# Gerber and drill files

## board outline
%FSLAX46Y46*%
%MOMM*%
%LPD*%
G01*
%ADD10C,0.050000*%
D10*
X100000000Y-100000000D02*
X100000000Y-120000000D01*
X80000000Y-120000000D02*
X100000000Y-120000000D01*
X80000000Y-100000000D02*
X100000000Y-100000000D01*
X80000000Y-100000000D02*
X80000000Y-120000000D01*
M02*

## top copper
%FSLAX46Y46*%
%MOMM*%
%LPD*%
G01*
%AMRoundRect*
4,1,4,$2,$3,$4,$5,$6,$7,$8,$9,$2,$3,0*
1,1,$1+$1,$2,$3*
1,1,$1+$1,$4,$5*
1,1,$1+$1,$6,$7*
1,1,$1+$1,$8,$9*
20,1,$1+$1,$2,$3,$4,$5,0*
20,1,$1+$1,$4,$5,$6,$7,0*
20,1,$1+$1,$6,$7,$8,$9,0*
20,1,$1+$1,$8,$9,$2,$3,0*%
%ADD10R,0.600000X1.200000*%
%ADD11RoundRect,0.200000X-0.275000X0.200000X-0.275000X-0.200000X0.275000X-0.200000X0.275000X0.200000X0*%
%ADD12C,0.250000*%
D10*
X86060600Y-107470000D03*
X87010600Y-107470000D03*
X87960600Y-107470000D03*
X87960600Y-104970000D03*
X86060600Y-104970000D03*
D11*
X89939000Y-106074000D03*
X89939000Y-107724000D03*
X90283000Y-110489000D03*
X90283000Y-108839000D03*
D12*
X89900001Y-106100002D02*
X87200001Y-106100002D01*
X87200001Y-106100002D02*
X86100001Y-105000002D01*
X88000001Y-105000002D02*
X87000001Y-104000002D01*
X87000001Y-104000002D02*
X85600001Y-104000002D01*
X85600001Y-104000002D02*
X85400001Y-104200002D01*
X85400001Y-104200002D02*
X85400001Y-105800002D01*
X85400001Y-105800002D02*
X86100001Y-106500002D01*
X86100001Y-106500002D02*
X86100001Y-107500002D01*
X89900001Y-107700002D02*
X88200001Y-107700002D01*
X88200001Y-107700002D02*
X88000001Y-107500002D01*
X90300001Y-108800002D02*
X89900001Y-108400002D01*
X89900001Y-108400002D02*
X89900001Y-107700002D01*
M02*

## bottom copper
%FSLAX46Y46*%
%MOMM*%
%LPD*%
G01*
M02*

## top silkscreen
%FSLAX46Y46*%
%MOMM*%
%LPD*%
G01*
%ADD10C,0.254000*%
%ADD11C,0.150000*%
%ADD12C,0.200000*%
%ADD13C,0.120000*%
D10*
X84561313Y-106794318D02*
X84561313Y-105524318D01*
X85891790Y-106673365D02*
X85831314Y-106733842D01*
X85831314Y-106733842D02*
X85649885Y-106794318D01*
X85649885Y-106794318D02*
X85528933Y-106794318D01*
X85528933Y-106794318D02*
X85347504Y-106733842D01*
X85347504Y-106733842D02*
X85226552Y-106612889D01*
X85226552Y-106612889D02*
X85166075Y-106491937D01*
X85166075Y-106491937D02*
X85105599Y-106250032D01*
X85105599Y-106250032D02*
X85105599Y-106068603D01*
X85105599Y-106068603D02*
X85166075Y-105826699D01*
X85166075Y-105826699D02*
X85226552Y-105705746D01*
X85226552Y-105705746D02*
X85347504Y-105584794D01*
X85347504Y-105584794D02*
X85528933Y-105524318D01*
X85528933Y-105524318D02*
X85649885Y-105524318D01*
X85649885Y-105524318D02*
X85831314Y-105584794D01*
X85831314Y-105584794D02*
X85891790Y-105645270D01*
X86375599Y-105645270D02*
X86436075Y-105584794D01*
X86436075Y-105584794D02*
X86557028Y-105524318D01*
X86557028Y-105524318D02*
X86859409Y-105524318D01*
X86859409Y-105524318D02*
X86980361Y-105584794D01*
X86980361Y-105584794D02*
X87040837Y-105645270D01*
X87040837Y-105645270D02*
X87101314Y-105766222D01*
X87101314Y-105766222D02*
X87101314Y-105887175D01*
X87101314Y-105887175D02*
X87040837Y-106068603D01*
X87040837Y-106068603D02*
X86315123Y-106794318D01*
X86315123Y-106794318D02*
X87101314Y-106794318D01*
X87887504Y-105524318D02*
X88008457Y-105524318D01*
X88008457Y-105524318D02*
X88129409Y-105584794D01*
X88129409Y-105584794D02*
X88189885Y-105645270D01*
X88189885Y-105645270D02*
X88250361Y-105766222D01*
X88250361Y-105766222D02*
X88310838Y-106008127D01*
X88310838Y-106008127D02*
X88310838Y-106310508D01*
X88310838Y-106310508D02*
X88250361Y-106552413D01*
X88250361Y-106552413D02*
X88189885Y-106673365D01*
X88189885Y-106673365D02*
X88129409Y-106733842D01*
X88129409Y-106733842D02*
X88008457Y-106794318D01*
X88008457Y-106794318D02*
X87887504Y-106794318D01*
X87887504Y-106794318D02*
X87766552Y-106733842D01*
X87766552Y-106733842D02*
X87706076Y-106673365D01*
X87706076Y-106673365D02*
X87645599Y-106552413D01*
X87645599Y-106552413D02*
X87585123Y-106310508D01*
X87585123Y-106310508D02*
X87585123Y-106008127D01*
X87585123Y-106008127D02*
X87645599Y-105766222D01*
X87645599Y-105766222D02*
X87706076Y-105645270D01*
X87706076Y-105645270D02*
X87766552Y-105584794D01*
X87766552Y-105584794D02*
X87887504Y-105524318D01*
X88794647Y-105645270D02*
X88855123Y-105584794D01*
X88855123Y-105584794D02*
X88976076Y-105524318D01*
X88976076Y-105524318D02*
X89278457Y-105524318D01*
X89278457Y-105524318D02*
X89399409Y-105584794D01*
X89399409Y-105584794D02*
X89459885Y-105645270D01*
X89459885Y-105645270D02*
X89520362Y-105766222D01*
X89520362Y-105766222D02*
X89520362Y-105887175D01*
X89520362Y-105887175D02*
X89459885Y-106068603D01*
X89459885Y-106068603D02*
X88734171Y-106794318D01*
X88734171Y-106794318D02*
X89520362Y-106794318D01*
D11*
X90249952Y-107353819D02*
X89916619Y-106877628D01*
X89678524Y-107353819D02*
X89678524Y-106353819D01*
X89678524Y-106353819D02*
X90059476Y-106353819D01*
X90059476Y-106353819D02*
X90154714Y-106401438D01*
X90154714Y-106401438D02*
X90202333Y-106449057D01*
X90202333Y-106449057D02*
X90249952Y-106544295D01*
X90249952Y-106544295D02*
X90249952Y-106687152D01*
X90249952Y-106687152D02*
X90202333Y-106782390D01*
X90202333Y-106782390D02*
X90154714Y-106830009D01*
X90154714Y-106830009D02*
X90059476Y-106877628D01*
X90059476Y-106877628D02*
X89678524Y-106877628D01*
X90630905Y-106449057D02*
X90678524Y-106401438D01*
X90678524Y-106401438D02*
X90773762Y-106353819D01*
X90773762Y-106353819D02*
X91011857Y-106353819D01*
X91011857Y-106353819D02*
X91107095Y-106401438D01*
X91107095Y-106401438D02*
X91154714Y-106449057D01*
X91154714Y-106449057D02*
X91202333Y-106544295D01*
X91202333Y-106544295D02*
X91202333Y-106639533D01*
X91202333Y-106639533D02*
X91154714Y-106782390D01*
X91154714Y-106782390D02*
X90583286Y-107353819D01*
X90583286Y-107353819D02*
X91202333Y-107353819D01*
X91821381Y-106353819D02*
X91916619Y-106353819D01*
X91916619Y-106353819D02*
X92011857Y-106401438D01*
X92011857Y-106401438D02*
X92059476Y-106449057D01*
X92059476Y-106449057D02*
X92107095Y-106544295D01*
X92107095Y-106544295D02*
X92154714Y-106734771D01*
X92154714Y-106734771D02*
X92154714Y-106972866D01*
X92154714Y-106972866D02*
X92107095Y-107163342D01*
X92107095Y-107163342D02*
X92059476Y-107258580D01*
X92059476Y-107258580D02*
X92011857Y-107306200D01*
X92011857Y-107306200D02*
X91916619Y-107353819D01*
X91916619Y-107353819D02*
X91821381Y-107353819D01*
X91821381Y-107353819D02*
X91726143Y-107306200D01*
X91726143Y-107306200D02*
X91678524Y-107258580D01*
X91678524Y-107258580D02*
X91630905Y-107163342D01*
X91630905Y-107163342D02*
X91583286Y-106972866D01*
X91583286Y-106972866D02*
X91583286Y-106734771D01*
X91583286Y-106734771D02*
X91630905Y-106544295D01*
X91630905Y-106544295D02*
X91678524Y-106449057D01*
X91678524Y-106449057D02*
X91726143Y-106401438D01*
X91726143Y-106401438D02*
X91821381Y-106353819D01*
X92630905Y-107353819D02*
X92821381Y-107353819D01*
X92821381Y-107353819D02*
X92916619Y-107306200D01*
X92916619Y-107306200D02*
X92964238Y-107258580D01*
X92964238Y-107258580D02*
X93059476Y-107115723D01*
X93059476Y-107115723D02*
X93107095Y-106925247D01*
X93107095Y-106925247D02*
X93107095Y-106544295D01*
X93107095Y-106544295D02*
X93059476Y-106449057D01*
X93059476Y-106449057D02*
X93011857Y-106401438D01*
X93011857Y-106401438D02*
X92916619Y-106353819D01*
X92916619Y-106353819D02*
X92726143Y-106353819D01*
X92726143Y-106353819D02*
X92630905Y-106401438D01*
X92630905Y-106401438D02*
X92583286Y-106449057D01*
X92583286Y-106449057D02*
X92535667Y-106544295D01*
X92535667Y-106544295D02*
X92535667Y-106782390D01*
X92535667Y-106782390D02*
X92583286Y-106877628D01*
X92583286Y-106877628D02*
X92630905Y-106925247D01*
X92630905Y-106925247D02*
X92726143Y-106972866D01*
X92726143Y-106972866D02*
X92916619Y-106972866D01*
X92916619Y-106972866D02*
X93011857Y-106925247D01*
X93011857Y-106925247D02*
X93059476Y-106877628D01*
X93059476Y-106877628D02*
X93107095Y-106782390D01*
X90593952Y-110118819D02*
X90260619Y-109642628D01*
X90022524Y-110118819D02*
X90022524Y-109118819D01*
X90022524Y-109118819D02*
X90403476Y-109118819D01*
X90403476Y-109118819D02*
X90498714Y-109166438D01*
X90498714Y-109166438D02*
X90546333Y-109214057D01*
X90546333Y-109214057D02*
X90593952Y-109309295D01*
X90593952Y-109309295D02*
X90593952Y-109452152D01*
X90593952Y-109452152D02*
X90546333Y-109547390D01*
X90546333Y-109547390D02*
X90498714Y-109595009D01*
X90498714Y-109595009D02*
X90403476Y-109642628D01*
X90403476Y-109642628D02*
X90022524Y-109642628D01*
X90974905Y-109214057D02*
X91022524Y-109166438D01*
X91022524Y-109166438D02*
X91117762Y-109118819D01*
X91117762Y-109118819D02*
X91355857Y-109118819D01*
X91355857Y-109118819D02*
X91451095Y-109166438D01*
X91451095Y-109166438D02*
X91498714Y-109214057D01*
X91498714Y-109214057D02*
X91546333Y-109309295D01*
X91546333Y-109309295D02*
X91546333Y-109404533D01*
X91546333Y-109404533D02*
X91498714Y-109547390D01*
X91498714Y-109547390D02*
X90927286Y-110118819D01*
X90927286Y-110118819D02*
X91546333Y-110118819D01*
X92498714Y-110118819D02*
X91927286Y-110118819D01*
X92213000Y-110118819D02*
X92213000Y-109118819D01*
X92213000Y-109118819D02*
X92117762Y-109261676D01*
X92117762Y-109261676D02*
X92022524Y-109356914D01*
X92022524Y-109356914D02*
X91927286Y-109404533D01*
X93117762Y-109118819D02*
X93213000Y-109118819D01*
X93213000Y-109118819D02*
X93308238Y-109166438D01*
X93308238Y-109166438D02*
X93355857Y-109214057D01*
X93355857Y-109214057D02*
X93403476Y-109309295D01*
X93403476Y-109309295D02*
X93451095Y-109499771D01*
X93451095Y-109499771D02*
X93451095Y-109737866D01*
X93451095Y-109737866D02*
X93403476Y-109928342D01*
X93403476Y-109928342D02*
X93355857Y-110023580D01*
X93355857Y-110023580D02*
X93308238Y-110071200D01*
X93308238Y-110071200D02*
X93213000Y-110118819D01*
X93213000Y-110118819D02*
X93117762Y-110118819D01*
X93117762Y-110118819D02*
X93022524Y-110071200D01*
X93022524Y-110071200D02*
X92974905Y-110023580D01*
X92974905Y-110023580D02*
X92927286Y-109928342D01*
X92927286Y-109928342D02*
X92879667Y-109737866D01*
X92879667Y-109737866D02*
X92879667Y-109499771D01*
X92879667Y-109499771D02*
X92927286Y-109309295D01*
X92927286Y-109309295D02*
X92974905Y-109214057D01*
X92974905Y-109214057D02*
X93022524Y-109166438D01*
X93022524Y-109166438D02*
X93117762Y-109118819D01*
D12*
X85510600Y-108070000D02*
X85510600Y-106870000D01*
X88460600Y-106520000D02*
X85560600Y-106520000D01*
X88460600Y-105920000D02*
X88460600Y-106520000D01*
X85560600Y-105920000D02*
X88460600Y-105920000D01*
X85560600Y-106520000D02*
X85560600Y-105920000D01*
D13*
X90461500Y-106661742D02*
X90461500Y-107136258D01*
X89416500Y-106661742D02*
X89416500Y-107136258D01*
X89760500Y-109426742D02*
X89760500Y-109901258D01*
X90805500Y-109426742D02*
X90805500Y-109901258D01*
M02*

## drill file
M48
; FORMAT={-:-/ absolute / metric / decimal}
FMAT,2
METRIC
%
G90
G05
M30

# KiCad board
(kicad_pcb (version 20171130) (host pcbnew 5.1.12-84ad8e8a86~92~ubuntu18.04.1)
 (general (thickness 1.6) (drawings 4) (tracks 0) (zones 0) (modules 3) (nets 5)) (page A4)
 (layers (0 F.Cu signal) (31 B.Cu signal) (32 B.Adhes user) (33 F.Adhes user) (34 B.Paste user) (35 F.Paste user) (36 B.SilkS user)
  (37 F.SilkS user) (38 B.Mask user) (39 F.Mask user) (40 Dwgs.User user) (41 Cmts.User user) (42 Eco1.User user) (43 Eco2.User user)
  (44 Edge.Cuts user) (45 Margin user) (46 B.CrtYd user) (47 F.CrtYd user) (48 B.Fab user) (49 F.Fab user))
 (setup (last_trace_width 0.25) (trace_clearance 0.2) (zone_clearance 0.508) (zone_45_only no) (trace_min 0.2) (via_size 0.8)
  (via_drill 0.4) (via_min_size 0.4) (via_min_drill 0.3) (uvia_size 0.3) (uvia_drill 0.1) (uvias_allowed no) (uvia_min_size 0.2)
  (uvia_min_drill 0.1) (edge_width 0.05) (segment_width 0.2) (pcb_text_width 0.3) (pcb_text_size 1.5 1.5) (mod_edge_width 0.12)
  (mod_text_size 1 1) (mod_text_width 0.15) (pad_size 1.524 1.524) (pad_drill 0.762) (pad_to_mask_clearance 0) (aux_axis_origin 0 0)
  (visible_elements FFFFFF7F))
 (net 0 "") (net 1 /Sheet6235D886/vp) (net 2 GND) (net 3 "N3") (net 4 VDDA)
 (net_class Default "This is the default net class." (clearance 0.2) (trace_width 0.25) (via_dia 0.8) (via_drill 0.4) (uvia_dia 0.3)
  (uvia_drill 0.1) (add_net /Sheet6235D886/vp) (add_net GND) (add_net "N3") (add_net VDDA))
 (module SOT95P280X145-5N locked (layer F.Cu) (at 87.010600 106.220000 90.000000)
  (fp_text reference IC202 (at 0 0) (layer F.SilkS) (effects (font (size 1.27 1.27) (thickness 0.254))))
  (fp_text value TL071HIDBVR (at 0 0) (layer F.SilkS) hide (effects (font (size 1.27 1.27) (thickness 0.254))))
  (fp_line (start -1.85 -1.5) (end -0.65 -1.5) (layer F.SilkS) (width 0.2))
  (fp_line (start -0.3 1.45) (end -0.3 -1.45) (layer F.SilkS) (width 0.2))
  (fp_line (start 0.3 1.45) (end -0.3 1.45) (layer F.SilkS) (width 0.2))
  (fp_line (start 0.3 -1.45) (end 0.3 1.45) (layer F.SilkS) (width 0.2))
  (fp_line (start -0.3 -1.45) (end 0.3 -1.45) (layer F.SilkS) (width 0.2))
  (pad 1 smd rect (at -1.25 -0.95 180.000000) (size 0.6 1.2) (layers F.Cu F.Mask F.Paste) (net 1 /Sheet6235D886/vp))
  (pad 2 smd rect (at -1.25 0 180.000000) (size 0.6 1.2) (layers F.Cu F.Mask F.Paste) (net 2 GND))
  (pad 3 smd rect (at -1.25 0.95 180.000000) (size 0.6 1.2) (layers F.Cu F.Mask F.Paste) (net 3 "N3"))
  (pad 4 smd rect (at 1.25 0.95 180.000000) (size 0.6 1.2) (layers F.Cu F.Mask F.Paste) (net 1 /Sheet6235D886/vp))
  (pad 5 smd rect (at 1.25 -0.95 180.000000) (size 0.6 1.2) (layers F.Cu F.Mask F.Paste) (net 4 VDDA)))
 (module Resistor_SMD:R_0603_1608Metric (layer F.Cu) (at 89.939000 106.899000 270.000000)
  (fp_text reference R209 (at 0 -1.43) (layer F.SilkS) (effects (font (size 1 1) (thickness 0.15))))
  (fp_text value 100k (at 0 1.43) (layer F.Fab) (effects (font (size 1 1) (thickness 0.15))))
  (fp_line (start -0.237258 -0.5225) (end 0.237258 -0.5225) (layer F.SilkS) (width 0.12))
  (fp_line (start -0.237258 0.5225) (end 0.237258 0.5225) (layer F.SilkS) (width 0.12))
  (pad 1 smd roundrect (at -0.825 0 270.000000) (size 0.8 0.95) (layers F.Cu F.Mask F.Paste) (roundrect_rratio 0.25) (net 4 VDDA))
  (pad 2 smd roundrect (at 0.825 0 270.000000) (size 0.8 0.95) (layers F.Cu F.Mask F.Paste) (roundrect_rratio 0.25) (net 3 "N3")))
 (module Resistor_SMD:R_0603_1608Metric (layer F.Cu) (at 90.283000 109.664000 270.000000)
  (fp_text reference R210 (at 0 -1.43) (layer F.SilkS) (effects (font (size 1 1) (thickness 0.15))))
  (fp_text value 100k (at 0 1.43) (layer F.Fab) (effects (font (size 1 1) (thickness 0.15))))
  (fp_line (start -0.237258 0.5225) (end 0.237258 0.5225) (layer F.SilkS) (width 0.12))
  (fp_line (start -0.237258 -0.5225) (end 0.237258 -0.5225) (layer F.SilkS) (width 0.12))
  (pad 2 smd roundrect (at 0.825 0 270.000000) (size 0.8 0.95) (layers F.Cu F.Mask F.Paste) (roundrect_rratio 0.25) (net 2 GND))
  (pad 1 smd roundrect (at -0.825 0 270.000000) (size 0.8 0.95) (layers F.Cu F.Mask F.Paste) (roundrect_rratio 0.25) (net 3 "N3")))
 (gr_line (start 100 100) (end 100 120) (layer Edge.Cuts) (width 0.05))
 (gr_line (start 80 120) (end 100 120) (layer Edge.Cuts) (width 0.05))
 (gr_line (start 80 100) (end 100 100) (layer Edge.Cuts) (width 0.05))
 (gr_line (start 80 100) (end 80 120) (layer Edge.Cuts) (width 0.05))
 (segment (start 89.900001 106.100002) (end 87.200001 106.100002) (width 0.250000) (layer F.Cu) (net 4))
 (segment (start 87.200001 106.100002) (end 86.100001 105.000002) (width 0.250000) (layer F.Cu) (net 4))
 (segment (start 88.000001 105.000002) (end 87.000001 104.000002) (width 0.250000) (layer F.Cu) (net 1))
 (segment (start 87.000001 104.000002) (end 85.600001 104.000002) (width 0.250000) (layer F.Cu) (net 1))
 (segment (start 85.600001 104.000002) (end 85.400001 104.200002) (width 0.250000) (layer F.Cu) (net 1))
 (segment (start 85.400001 104.200002) (end 85.400001 105.800002) (width 0.250000) (layer F.Cu) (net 1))
 (segment (start 85.400001 105.800002) (end 86.100001 106.500002) (width 0.250000) (layer F.Cu) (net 1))
 (segment (start 86.100001 106.500002) (end 86.100001 107.500002) (width 0.250000) (layer F.Cu) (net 1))
 (segment (start 89.900001 107.700002) (end 88.200001 107.700002) (width 0.250000) (layer F.Cu) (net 3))
 (segment (start 88.200001 107.700002) (end 88.000001 107.500002) (width 0.250000) (layer F.Cu) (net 3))
 (segment (start 90.300001 108.800002) (end 89.900001 108.400002) (width 0.250000) (layer F.Cu) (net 3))
 (segment (start 89.900001 108.400002) (end 89.900001 107.700002) (width 0.250000) (layer F.Cu) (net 3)))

